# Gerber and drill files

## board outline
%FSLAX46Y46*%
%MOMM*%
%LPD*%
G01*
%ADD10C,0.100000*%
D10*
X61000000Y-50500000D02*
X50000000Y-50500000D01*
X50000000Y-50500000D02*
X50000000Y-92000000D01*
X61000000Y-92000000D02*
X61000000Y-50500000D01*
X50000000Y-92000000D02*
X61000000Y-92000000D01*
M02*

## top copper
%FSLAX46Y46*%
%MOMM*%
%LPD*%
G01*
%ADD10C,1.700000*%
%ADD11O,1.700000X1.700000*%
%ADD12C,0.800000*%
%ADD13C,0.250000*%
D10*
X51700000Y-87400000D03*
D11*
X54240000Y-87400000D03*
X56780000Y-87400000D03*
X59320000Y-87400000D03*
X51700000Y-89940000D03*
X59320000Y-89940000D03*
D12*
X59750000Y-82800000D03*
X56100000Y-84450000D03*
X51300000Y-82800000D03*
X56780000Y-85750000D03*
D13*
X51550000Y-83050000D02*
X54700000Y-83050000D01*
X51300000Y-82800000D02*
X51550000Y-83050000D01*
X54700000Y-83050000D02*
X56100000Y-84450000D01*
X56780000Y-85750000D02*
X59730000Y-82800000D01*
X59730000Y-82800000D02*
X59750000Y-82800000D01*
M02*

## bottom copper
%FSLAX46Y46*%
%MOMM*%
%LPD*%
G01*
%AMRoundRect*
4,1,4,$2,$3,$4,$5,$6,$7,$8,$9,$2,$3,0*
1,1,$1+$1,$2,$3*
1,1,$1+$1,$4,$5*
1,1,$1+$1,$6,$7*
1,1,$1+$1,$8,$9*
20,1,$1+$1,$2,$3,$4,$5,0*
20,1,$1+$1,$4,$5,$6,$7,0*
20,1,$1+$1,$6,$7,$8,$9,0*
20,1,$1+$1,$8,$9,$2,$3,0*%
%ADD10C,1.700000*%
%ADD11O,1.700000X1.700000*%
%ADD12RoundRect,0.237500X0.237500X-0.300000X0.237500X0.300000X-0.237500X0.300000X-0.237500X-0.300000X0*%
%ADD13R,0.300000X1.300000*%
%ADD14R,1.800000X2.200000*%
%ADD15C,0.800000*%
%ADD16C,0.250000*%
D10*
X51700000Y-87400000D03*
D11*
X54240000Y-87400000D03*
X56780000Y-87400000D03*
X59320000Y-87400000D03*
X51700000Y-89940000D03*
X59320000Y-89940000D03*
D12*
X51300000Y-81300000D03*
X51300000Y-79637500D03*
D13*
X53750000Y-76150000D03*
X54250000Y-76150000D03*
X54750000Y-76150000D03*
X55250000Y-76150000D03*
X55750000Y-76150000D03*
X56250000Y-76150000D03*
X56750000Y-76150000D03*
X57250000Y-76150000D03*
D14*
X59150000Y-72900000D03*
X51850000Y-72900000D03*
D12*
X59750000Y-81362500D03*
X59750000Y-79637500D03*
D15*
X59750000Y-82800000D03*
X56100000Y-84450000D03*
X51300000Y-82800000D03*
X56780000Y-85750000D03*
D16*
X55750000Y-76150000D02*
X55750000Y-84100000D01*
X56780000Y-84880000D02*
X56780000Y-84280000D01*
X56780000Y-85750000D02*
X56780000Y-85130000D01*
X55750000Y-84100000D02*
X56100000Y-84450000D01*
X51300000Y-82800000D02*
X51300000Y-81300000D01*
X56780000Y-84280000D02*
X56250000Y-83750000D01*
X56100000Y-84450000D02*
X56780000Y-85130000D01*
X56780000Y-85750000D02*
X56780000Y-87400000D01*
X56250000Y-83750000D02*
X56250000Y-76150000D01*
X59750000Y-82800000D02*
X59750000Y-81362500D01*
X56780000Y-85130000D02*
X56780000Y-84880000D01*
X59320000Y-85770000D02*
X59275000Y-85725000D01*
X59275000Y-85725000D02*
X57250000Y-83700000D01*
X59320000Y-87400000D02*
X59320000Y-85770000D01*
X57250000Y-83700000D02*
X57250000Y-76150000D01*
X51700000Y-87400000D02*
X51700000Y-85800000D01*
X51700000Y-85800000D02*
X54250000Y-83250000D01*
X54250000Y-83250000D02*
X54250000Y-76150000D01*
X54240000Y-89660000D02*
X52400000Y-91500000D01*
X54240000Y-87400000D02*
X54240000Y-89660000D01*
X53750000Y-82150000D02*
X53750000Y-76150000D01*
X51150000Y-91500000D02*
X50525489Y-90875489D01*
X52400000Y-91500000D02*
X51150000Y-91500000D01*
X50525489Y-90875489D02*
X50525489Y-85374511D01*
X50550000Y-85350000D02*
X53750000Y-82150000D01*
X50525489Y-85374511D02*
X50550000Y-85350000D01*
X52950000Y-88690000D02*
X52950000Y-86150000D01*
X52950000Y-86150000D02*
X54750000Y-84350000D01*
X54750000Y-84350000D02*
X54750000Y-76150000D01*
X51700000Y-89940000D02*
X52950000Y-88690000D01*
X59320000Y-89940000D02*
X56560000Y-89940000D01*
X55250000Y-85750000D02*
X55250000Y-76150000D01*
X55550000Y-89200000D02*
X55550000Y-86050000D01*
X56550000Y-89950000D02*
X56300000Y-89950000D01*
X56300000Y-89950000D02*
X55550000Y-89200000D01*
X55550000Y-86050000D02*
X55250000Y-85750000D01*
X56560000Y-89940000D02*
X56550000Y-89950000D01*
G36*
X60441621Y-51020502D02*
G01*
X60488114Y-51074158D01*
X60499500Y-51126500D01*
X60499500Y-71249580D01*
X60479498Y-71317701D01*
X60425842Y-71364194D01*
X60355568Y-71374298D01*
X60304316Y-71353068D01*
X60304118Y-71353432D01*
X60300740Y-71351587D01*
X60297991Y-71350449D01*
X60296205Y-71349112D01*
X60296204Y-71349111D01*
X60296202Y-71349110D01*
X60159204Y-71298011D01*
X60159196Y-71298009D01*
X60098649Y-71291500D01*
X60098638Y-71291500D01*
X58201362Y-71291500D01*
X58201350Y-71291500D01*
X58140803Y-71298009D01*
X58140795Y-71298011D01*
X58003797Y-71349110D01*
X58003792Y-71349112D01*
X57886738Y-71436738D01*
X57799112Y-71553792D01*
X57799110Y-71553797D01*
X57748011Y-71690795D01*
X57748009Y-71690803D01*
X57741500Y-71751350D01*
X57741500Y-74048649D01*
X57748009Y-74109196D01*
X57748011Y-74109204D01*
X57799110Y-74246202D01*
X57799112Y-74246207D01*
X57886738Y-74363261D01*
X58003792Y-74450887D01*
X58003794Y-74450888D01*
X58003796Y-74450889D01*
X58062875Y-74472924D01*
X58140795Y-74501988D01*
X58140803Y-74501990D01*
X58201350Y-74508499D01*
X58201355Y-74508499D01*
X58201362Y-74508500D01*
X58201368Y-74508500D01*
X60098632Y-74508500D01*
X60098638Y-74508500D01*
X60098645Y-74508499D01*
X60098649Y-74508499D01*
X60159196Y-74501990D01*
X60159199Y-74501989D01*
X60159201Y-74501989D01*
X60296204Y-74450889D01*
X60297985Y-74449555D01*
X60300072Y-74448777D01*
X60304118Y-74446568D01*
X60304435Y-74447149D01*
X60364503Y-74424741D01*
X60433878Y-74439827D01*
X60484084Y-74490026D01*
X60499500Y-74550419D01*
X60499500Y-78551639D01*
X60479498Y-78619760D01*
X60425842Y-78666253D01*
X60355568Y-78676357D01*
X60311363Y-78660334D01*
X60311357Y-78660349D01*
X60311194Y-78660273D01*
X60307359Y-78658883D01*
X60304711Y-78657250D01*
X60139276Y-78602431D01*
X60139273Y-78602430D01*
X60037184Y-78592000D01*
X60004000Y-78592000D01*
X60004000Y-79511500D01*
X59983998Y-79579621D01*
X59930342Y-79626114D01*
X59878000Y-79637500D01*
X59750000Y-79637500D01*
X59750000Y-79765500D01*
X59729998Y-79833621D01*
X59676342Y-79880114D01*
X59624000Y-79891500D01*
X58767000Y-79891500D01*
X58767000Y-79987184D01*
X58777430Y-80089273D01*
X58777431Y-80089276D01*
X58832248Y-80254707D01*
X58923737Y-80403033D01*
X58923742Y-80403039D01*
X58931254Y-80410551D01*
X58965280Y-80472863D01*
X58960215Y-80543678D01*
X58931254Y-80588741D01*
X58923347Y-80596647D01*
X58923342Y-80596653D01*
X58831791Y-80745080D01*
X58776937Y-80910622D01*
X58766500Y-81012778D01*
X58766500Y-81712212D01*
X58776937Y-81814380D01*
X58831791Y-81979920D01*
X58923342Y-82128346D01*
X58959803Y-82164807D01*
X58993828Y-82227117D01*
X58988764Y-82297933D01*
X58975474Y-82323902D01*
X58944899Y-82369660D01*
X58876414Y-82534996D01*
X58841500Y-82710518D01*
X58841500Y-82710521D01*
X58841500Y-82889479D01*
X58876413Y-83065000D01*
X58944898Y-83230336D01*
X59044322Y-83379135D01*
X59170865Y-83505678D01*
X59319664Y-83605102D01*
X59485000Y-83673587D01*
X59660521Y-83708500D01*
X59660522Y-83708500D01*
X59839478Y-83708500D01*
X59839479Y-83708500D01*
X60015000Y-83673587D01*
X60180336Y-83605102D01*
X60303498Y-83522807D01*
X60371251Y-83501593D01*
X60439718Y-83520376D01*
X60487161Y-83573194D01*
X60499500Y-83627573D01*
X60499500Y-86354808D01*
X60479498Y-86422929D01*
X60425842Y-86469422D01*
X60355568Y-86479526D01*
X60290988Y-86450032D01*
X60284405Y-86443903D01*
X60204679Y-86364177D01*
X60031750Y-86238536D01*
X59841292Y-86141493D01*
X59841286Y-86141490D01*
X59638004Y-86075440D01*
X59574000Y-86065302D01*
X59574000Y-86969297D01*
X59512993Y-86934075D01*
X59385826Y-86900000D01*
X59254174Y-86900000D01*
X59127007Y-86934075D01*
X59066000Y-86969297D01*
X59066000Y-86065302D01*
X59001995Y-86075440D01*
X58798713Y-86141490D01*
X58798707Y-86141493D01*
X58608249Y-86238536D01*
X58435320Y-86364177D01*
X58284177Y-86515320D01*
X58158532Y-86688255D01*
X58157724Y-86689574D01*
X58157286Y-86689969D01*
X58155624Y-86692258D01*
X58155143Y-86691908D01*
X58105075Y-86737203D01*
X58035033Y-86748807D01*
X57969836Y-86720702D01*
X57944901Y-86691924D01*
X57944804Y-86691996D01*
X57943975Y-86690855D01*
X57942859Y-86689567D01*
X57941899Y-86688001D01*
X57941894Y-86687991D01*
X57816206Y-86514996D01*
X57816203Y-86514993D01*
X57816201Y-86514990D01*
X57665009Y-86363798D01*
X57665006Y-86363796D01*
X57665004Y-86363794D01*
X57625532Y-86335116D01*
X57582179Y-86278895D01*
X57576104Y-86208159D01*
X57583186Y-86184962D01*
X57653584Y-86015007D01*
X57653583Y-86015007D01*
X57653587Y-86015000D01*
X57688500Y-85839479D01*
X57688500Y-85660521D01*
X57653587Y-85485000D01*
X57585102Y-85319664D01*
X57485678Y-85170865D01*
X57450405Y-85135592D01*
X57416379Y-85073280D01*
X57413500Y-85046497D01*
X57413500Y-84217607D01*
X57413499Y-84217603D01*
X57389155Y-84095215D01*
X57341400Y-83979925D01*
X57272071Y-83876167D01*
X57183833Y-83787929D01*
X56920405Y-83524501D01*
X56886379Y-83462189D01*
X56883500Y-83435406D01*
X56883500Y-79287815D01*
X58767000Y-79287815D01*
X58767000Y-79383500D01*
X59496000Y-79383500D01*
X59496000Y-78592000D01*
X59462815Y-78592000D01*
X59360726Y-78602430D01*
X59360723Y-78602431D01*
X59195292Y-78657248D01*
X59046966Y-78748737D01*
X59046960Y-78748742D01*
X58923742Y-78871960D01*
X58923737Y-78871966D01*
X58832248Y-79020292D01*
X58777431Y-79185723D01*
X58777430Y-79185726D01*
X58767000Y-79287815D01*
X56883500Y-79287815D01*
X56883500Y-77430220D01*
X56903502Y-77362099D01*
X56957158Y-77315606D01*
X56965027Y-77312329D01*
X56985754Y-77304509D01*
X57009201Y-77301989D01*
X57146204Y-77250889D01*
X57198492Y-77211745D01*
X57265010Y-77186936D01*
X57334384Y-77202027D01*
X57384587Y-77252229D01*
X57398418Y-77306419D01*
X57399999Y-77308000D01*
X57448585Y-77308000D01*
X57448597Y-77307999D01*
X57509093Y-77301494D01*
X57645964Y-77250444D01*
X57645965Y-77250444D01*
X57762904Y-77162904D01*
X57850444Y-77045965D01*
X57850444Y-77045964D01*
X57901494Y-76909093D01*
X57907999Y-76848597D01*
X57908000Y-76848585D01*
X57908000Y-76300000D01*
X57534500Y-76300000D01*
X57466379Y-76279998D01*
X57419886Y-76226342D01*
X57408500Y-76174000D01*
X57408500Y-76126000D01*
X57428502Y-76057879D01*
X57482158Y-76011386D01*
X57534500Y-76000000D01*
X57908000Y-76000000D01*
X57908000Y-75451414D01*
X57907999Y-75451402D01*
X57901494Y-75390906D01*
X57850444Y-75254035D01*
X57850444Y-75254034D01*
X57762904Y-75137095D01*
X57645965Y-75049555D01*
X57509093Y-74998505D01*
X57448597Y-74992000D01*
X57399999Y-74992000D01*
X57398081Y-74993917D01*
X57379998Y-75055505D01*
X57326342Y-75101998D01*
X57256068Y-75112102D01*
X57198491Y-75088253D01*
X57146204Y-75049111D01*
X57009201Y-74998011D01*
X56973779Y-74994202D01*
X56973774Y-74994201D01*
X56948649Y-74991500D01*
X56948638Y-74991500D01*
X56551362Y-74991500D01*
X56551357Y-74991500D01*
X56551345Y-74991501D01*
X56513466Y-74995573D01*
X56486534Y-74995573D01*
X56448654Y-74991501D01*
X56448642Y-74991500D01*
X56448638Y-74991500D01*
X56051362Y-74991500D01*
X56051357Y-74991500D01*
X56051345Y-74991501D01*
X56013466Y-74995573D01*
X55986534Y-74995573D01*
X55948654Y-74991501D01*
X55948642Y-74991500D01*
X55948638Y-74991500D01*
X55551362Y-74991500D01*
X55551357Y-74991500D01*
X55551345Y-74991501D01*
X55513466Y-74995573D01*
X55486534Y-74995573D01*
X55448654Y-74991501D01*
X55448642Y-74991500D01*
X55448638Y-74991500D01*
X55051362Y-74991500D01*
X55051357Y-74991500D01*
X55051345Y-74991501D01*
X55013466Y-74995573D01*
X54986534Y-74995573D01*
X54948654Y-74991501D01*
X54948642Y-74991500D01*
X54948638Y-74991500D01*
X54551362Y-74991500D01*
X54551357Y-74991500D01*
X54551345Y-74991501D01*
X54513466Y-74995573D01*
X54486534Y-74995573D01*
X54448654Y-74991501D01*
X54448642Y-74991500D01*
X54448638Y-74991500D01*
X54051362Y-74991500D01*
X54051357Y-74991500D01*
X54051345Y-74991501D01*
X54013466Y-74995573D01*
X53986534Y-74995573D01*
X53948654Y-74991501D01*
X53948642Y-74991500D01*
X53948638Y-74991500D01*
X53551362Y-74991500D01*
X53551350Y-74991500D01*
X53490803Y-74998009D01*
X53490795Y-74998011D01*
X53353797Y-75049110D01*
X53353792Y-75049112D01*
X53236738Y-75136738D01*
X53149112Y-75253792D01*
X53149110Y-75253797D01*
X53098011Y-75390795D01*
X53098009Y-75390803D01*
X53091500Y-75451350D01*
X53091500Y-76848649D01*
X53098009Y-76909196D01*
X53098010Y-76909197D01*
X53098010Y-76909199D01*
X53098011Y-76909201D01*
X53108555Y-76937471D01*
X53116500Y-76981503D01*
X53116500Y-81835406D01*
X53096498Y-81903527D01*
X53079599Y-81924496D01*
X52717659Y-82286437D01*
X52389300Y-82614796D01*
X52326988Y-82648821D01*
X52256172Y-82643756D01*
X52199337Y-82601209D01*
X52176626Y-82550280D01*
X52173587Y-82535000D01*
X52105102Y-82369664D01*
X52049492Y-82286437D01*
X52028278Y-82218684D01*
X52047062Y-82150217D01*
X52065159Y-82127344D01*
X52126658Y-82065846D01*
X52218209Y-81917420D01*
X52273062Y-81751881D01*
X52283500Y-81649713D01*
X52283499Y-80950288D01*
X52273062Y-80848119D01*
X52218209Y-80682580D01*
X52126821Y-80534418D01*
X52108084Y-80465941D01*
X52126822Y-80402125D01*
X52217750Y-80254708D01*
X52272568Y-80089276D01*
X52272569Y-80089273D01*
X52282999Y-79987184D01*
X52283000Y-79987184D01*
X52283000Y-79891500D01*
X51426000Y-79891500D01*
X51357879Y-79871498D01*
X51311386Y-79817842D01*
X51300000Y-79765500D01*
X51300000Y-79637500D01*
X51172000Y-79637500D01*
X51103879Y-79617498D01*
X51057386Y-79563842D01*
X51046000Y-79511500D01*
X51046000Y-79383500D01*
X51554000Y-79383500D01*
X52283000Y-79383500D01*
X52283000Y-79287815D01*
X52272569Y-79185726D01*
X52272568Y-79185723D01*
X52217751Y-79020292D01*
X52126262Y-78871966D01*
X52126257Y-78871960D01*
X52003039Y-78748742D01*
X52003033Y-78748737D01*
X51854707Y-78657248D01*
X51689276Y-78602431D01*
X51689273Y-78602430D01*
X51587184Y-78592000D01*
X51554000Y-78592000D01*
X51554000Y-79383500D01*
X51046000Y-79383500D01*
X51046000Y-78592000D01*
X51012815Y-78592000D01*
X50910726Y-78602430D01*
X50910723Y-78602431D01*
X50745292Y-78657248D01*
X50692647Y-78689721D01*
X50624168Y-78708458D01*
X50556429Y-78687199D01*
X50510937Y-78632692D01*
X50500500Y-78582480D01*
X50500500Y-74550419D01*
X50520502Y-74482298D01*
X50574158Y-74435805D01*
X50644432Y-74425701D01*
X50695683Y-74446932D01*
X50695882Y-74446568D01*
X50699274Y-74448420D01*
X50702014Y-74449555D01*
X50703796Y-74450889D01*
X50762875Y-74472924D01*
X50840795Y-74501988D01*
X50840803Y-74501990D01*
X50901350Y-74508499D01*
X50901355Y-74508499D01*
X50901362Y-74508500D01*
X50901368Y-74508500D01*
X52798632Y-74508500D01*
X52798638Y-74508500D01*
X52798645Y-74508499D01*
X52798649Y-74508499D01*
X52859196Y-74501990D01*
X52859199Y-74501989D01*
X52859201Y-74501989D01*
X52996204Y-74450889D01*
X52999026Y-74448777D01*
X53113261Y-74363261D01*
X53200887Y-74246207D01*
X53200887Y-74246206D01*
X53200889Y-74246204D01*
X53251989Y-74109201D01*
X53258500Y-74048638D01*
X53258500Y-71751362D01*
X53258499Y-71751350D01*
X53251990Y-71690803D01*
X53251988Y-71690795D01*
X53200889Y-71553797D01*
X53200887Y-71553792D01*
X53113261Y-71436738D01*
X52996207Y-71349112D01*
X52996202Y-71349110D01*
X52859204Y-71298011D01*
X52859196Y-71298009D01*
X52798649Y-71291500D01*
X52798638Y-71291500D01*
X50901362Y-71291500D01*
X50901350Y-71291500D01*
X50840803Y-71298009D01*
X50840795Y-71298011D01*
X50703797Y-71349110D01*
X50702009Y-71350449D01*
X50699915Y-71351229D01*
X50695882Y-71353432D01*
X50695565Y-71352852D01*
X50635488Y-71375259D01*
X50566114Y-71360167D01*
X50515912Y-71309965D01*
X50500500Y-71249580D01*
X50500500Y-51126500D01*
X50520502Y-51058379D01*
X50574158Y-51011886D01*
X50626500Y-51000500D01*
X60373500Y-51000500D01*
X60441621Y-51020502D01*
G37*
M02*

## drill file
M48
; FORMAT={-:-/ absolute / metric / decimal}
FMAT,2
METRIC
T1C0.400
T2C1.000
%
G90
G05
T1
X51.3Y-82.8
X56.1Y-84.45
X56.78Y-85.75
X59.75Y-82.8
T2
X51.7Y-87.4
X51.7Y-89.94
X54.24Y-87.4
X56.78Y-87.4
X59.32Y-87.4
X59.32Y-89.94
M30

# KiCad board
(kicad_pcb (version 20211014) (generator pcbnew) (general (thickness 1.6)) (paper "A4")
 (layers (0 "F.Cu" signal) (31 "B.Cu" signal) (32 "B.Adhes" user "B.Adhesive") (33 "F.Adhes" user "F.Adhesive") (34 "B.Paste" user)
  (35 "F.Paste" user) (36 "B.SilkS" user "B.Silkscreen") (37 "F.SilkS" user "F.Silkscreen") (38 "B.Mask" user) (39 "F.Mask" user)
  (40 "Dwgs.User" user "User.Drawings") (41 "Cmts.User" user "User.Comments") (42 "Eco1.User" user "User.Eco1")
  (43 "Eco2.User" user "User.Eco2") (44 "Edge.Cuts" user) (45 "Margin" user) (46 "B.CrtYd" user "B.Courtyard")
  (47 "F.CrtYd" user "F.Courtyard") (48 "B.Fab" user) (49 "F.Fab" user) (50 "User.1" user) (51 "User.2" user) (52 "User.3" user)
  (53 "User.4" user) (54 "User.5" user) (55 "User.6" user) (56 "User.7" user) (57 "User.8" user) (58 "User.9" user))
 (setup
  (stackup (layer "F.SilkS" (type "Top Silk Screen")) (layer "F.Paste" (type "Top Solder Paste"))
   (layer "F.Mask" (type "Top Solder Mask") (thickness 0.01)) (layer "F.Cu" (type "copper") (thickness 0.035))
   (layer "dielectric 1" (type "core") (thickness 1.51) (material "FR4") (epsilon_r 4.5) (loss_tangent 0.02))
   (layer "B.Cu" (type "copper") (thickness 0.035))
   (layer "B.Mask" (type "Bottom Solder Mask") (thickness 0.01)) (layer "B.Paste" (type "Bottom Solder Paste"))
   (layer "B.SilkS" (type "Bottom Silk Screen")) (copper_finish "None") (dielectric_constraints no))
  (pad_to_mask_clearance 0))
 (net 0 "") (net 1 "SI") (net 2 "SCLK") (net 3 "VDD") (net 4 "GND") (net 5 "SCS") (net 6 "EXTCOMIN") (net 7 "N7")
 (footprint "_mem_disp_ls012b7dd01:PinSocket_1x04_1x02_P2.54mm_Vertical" (layer "F.Cu") (at 51.7 87.4 90)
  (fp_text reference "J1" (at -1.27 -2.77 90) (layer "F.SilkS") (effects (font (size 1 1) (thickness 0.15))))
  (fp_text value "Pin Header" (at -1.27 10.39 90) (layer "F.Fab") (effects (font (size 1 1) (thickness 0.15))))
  (pad "1" thru_hole circle (at 0 0 90) (size 1.7 1.7) (drill 1) (layers *.Cu *.Mask) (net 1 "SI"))
  (pad "2" thru_hole oval (at 0 2.54 90) (size 1.7 1.7) (drill 1) (layers *.Cu *.Mask) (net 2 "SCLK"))
  (pad "3" thru_hole oval (at 0 5.08 90) (size 1.7 1.7) (drill 1) (layers *.Cu *.Mask) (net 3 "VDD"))
  (pad "4" thru_hole oval (at 0 7.62 90) (size 1.7 1.7) (drill 1) (layers *.Cu *.Mask) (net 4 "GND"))
  (pad "5" thru_hole oval (at -2.54 0 90) (size 1.7 1.7) (drill 1) (layers *.Cu *.Mask) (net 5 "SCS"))
  (pad "6" thru_hole oval (at -2.54 7.62 90) (size 1.7 1.7) (drill 1) (layers *.Cu *.Mask) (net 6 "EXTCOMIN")))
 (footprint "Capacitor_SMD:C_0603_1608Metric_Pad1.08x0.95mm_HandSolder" (layer "B.Cu") (at 51.3 80.5 90)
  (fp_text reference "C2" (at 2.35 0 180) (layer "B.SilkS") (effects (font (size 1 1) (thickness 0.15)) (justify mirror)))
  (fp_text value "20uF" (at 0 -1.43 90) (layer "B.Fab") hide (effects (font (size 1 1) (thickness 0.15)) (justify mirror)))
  (pad "1" smd roundrect (at -0.8 0 90) (size 1.075 0.95) (layers "B.Cu" "B.Paste" "B.Mask") (roundrect_rratio 0.25) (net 3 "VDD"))
  (pad "2" smd roundrect (at 0.8625 0 90) (size 1.075 0.95) (layers "B.Cu" "B.Paste" "B.Mask") (roundrect_rratio 0.25) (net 4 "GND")))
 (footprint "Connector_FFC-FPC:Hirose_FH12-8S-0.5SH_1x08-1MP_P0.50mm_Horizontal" (layer "B.Cu") (at 55.5 74.3)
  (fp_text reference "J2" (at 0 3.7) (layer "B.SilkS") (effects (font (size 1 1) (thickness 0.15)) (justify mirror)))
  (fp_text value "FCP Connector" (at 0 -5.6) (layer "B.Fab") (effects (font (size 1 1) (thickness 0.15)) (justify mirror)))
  (pad "1" smd rect (at -1.75 1.85) (size 0.3 1.3) (layers "B.Cu" "B.Paste" "B.Mask") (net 2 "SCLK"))
  (pad "2" smd rect (at -1.25 1.85) (size 0.3 1.3) (layers "B.Cu" "B.Paste" "B.Mask") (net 1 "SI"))
  (pad "3" smd rect (at -0.75 1.85) (size 0.3 1.3) (layers "B.Cu" "B.Paste" "B.Mask") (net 5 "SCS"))
  (pad "4" smd rect (at -0.25 1.85) (size 0.3 1.3) (layers "B.Cu" "B.Paste" "B.Mask") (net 6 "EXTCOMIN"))
  (pad "5" smd rect (at 0.25 1.85) (size 0.3 1.3) (layers "B.Cu" "B.Paste" "B.Mask") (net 3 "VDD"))
  (pad "6" smd rect (at 0.75 1.85) (size 0.3 1.3) (layers "B.Cu" "B.Paste" "B.Mask") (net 3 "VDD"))
  (pad "7" smd rect (at 1.25 1.85) (size 0.3 1.3) (layers "B.Cu" "B.Paste" "B.Mask") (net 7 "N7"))
  (pad "8" smd rect (at 1.75 1.85) (size 0.3 1.3) (layers "B.Cu" "B.Paste" "B.Mask") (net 4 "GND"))
  (pad "MP" smd rect (at 3.65 -1.4) (size 1.8 2.2) (layers "B.Cu" "B.Paste" "B.Mask"))
  (pad "MP" smd rect (at -3.65 -1.4) (size 1.8 2.2) (layers "B.Cu" "B.Paste" "B.Mask")))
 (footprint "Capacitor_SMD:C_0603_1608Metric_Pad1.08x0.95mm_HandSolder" (layer "B.Cu") (at 59.75 80.5 90)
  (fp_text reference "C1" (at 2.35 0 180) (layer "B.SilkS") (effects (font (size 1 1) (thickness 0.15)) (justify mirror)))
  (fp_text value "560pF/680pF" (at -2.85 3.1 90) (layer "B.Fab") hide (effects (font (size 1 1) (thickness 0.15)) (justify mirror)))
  (pad "1" smd roundrect (at -0.8625 0 90) (size 1.075 0.95) (layers "B.Cu" "B.Paste" "B.Mask") (roundrect_rratio 0.25) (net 3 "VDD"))
  (pad "2" smd roundrect (at 0.8625 0 90) (size 1.075 0.95) (layers "B.Cu" "B.Paste" "B.Mask") (roundrect_rratio 0.25) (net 4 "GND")))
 (gr_line (start 61 50.5) (end 50 50.5) (layer "Edge.Cuts") (width 0.1))
 (gr_line (start 50 50.5) (end 50 92) (layer "Edge.Cuts") (width 0.1))
 (gr_line (start 61 92) (end 61 50.5) (layer "Edge.Cuts") (width 0.1))
 (gr_line (start 50 92) (end 61 92) (layer "Edge.Cuts") (width 0.1))
 (segment (start 51.55 83.05) (end 54.7 83.05) (width 0.25) (layer "F.Cu") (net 3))
 (segment (start 51.3 82.8) (end 51.55 83.05) (width 0.25) (layer "F.Cu") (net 3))
 (segment (start 54.7 83.05) (end 56.1 84.45) (width 0.25) (layer "F.Cu") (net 3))
 (segment (start 56.78 85.75) (end 59.73 82.8) (width 0.25) (layer "F.Cu") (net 3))
 (segment (start 59.73 82.8) (end 59.75 82.8) (width 0.25) (layer "F.Cu") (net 3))
 (via (at 59.75 82.8) (size 0.8) (drill 0.4) (layers "F.Cu" "B.Cu") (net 3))
 (via (at 56.1 84.45) (size 0.8) (drill 0.4) (layers "F.Cu" "B.Cu") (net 3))
 (via (at 51.3 82.8) (size 0.8) (drill 0.4) (layers "F.Cu" "B.Cu") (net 3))
 (via (at 56.78 85.75) (size 0.8) (drill 0.4) (layers "F.Cu" "B.Cu") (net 3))
 (segment (start 55.75 76.15) (end 55.75 84.1) (width 0.25) (layer "B.Cu") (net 3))
 (segment (start 56.78 84.88) (end 56.78 84.28) (width 0.25) (layer "B.Cu") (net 3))
 (segment (start 56.78 85.75) (end 56.78 85.13) (width 0.25) (layer "B.Cu") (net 3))
 (segment (start 55.75 84.1) (end 56.1 84.45) (width 0.25) (layer "B.Cu") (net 3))
 (segment (start 51.3 82.8) (end 51.3 81.3) (width 0.25) (layer "B.Cu") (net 3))
 (segment (start 56.78 84.28) (end 56.25 83.75) (width 0.25) (layer "B.Cu") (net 3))
 (segment (start 56.1 84.45) (end 56.78 85.13) (width 0.25) (layer "B.Cu") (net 3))
 (segment (start 56.78 85.75) (end 56.78 87.4) (width 0.25) (layer "B.Cu") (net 3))
 (segment (start 56.25 83.75) (end 56.25 76.15) (width 0.25) (layer "B.Cu") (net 3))
 (segment (start 59.75 82.8) (end 59.75 81.3625) (width 0.25) (layer "B.Cu") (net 3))
 (segment (start 56.78 85.13) (end 56.78 84.88) (width 0.25) (layer "B.Cu") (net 3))
 (segment (start 59.32 85.77) (end 59.275 85.725) (width 0.25) (layer "B.Cu") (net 4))
 (segment (start 59.275 85.725) (end 57.25 83.7) (width 0.25) (layer "B.Cu") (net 4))
 (segment (start 59.32 87.4) (end 59.32 85.77) (width 0.25) (layer "B.Cu") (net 4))
 (segment (start 57.25 83.7) (end 57.25 76.15) (width 0.25) (layer "B.Cu") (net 4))
 (segment (start 51.7 87.4) (end 51.7 85.8) (width 0.25) (layer "B.Cu") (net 1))
 (segment (start 51.7 85.8) (end 54.25 83.25) (width 0.25) (layer "B.Cu") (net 1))
 (segment (start 54.25 83.25) (end 54.25 76.15) (width 0.25) (layer "B.Cu") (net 1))
 (segment (start 54.24 89.66) (end 52.4 91.5) (width 0.25) (layer "B.Cu") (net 2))
 (segment (start 54.24 87.4) (end 54.24 89.66) (width 0.25) (layer "B.Cu") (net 2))
 (segment (start 53.75 82.15) (end 53.75 76.15) (width 0.25) (layer "B.Cu") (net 2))
 (segment (start 51.15 91.5) (end 50.525489 90.875489) (width 0.25) (layer "B.Cu") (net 2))
 (segment (start 52.4 91.5) (end 51.15 91.5) (width 0.25) (layer "B.Cu") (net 2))
 (segment (start 50.525489 90.875489) (end 50.525489 85.374511) (width 0.25) (layer "B.Cu") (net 2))
 (segment (start 50.55 85.35) (end 53.75 82.15) (width 0.25) (layer "B.Cu") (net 2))
 (segment (start 50.525489 85.374511) (end 50.55 85.35) (width 0.25) (layer "B.Cu") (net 2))
 (segment (start 52.95 88.69) (end 52.95 86.15) (width 0.25) (layer "B.Cu") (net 5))
 (segment (start 52.95 86.15) (end 54.75 84.35) (width 0.25) (layer "B.Cu") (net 5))
 (segment (start 54.75 84.35) (end 54.75 76.15) (width 0.25) (layer "B.Cu") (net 5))
 (segment (start 51.7 89.94) (end 52.95 88.69) (width 0.25) (layer "B.Cu") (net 5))
 (segment (start 59.32 89.94) (end 56.56 89.94) (width 0.25) (layer "B.Cu") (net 6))
 (segment (start 55.25 85.75) (end 55.25 76.15) (width 0.25) (layer "B.Cu") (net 6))
 (segment (start 55.55 89.2) (end 55.55 86.05) (width 0.25) (layer "B.Cu") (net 6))
 (segment (start 56.55 89.95) (end 56.3 89.95) (width 0.25) (layer "B.Cu") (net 6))
 (segment (start 56.3 89.95) (end 55.55 89.2) (width 0.25) (layer "B.Cu") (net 6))
 (segment (start 55.55 86.05) (end 55.25 85.75) (width 0.25) (layer "B.Cu") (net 6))
 (segment (start 56.56 89.94) (end 56.55 89.95) (width 0.25) (layer "B.Cu") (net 6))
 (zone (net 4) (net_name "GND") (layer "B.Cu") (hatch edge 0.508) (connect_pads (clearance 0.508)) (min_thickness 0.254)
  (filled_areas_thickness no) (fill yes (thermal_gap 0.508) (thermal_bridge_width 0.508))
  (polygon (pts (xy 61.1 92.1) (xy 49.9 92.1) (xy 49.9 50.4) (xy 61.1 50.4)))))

